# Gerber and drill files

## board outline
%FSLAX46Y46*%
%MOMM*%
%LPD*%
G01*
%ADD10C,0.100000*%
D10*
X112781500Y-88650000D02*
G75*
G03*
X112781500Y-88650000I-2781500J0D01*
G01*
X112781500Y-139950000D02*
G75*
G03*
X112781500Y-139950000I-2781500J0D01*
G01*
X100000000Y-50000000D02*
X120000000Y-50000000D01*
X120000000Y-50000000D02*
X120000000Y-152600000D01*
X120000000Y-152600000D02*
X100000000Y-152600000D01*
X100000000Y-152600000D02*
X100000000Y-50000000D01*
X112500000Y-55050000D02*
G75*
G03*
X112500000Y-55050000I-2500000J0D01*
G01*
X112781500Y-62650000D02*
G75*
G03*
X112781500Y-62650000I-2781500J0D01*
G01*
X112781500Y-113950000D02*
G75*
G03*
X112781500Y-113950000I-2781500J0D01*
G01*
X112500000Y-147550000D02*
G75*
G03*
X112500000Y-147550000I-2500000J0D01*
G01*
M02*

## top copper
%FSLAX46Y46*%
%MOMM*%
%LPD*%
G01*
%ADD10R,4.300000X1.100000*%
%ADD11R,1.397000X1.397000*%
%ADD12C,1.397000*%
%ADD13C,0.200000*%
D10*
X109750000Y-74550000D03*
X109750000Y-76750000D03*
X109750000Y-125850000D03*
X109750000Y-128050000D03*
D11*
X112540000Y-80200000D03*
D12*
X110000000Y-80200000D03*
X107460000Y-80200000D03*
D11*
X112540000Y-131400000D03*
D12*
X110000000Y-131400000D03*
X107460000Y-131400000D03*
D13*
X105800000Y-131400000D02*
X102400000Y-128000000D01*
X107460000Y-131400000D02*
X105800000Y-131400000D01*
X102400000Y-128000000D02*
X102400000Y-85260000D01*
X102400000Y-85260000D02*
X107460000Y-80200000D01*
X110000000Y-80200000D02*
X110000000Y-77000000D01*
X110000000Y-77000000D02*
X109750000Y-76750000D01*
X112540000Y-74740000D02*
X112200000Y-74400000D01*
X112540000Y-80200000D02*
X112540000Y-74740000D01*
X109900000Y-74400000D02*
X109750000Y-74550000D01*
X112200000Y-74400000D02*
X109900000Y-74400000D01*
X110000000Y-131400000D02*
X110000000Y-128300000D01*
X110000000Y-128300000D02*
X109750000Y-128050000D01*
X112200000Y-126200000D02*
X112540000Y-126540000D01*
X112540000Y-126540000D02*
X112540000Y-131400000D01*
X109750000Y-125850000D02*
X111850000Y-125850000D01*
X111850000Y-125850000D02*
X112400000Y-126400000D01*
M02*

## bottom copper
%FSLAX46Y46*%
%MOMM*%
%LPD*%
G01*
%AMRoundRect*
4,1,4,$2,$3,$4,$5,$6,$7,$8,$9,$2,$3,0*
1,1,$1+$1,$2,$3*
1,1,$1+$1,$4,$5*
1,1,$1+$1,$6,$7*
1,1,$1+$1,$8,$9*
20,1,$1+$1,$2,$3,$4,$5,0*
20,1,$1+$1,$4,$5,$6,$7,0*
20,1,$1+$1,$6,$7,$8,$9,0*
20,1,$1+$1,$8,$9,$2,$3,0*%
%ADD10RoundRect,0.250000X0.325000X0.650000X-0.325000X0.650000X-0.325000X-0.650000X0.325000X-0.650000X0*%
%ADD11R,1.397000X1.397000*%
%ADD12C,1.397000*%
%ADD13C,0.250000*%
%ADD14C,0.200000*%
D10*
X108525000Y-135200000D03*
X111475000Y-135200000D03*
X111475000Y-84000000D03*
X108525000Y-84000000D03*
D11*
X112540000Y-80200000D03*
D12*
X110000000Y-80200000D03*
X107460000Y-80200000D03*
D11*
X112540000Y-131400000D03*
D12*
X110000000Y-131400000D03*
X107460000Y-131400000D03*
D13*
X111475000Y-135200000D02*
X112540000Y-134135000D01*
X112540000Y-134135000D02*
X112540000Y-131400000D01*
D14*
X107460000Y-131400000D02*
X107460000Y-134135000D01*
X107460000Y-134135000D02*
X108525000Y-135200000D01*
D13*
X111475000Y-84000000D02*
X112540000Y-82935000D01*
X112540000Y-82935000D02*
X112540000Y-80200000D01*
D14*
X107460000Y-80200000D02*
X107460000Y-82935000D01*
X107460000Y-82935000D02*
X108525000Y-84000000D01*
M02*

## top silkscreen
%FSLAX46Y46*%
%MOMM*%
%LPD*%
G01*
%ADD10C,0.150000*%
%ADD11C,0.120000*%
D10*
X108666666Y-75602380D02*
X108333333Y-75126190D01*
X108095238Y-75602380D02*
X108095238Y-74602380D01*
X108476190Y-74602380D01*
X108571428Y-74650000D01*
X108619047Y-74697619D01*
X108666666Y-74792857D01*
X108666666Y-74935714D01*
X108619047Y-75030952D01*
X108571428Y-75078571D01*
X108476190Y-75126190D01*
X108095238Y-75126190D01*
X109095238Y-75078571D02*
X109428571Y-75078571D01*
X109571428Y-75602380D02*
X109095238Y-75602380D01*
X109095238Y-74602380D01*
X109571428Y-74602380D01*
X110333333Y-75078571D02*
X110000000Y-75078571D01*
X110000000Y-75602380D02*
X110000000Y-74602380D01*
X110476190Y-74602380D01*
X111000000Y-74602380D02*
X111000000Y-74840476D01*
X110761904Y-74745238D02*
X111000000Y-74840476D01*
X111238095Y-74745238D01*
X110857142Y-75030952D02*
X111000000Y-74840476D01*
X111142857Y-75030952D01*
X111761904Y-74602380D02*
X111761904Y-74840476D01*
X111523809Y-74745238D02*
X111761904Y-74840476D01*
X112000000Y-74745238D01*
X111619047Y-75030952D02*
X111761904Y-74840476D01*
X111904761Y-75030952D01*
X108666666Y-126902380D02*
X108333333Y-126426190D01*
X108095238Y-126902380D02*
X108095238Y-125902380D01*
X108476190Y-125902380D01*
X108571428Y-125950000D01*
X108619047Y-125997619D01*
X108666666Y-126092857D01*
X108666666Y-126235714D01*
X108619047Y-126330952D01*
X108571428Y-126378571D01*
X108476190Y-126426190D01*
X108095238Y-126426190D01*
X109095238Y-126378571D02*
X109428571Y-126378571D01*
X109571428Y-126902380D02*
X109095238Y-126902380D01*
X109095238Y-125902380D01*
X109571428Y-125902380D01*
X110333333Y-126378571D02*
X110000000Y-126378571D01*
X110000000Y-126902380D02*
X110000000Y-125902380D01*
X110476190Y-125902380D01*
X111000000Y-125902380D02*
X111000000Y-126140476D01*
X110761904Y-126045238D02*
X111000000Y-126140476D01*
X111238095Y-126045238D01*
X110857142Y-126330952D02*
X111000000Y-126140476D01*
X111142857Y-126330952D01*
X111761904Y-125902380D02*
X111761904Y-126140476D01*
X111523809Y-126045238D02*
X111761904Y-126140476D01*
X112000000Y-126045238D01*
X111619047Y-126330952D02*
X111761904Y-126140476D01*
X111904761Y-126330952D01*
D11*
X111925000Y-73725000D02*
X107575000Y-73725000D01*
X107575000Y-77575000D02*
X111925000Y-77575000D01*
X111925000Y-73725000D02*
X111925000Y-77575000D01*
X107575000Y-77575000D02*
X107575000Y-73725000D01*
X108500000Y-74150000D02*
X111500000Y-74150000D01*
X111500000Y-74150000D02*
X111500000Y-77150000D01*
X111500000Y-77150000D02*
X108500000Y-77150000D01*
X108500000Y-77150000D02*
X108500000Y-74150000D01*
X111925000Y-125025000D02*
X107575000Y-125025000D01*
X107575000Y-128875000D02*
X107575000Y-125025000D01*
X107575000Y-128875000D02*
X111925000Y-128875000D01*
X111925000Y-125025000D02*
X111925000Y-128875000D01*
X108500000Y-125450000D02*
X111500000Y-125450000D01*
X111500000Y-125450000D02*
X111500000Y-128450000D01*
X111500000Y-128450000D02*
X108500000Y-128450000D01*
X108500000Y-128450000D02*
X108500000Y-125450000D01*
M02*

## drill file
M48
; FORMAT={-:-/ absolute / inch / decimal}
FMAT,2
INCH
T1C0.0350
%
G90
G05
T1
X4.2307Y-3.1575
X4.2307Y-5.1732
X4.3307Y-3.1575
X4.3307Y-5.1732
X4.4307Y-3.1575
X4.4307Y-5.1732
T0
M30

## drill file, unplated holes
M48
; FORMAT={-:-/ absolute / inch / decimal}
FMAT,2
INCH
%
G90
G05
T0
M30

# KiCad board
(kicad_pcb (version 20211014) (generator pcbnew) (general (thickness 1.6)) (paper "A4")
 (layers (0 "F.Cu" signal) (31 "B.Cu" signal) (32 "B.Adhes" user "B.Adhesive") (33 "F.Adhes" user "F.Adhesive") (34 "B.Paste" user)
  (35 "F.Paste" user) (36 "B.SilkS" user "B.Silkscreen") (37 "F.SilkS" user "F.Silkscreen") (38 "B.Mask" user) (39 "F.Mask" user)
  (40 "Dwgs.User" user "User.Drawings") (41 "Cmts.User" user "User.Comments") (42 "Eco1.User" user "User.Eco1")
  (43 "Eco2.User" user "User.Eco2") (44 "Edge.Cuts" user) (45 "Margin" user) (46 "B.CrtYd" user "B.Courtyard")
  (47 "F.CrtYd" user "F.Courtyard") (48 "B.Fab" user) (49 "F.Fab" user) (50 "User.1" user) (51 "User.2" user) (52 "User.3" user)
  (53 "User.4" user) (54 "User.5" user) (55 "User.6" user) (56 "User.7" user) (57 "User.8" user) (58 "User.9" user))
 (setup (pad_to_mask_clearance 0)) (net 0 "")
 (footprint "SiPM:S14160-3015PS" (layer "F.Cu") (at 110 75.65)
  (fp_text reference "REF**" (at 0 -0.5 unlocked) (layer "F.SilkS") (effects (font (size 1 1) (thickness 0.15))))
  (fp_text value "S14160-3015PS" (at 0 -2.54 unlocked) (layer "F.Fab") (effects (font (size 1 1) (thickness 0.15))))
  (fp_line (start 1.925 -1.925) (end -2.425 -1.925) (layer "F.SilkS") (width 0.12))
  (fp_line (start -2.425 1.925) (end 1.925 1.925) (layer "F.SilkS") (width 0.12))
  (fp_line (start 1.925 -1.925) (end 1.925 1.925) (layer "F.SilkS") (width 0.12))
  (fp_line (start -2.425 1.925) (end -2.425 -1.925) (layer "F.SilkS") (width 0.12))
  (fp_rect (start -1.5 -1.5) (end 1.5 1.5) (layer "F.SilkS") (width 0.12) (fill none))
  (pad "1" smd rect (at -0.25 -1.1) (size 4.3 1.1) (layers "F.Cu" "F.Paste" "F.Mask"))
  (pad "2" smd rect (at -0.25 1.1) (size 4.3 1.1) (layers "F.Cu" "F.Paste" "F.Mask")))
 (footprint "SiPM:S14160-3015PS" (layer "F.Cu") (at 110 126.95)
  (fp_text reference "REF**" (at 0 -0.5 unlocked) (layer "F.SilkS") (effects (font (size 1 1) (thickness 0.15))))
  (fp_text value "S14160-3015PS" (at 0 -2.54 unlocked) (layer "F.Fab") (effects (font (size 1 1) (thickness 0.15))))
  (fp_line (start 1.925 -1.925) (end -2.425 -1.925) (layer "F.SilkS") (width 0.12))
  (fp_line (start -2.425 1.925) (end -2.425 -1.925) (layer "F.SilkS") (width 0.12))
  (fp_line (start -2.425 1.925) (end 1.925 1.925) (layer "F.SilkS") (width 0.12))
  (fp_line (start 1.925 -1.925) (end 1.925 1.925) (layer "F.SilkS") (width 0.12))
  (fp_rect (start -1.5 -1.5) (end 1.5 1.5) (layer "F.SilkS") (width 0.12) (fill none))
  (pad "1" smd rect (at -0.25 -1.1) (size 4.3 1.1) (layers "F.Cu" "F.Paste" "F.Mask"))
  (pad "2" smd rect (at -0.25 1.1) (size 4.3 1.1) (layers "F.Cu" "F.Paste" "F.Mask")))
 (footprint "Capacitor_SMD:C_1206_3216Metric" (layer "B.Cu") (at 110 84 180)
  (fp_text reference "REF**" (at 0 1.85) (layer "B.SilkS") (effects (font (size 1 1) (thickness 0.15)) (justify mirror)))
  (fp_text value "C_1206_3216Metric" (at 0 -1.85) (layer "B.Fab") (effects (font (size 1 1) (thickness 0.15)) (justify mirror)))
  (pad "1" smd roundrect (at -1.475 0 180) (size 1.15 1.8) (layers "B.Cu" "B.Paste" "B.Mask") (roundrect_rratio 0.2173913043))
  (pad "2" smd roundrect (at 1.475 0 180) (size 1.15 1.8) (layers "B.Cu" "B.Paste" "B.Mask") (roundrect_rratio 0.2173913043)))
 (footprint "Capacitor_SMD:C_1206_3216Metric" (layer "B.Cu") (at 110 135.2 180)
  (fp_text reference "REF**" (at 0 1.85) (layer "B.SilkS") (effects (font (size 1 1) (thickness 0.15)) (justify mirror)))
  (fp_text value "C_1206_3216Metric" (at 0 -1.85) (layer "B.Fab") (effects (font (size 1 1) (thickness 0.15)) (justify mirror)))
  (pad "1" smd roundrect (at -1.475 0 180) (size 1.15 1.8) (layers "B.Cu" "B.Paste" "B.Mask") (roundrect_rratio 0.2173913043))
  (pad "2" smd roundrect (at 1.475 0 180) (size 1.15 1.8) (layers "B.Cu" "B.Paste" "B.Mask") (roundrect_rratio 0.2173913043)))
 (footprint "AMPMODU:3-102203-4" (layer "B.Cu") (at 112.54 80.2 180)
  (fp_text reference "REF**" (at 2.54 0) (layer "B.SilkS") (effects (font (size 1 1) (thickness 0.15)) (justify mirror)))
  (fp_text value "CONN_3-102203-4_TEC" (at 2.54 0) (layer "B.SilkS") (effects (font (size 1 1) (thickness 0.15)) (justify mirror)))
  (pad "1" thru_hole rect locked (at 0 0 180) (size 1.397 1.397) (drill 0.889) (layers *.Cu *.Mask))
  (pad "2" thru_hole circle locked (at 2.54 0 180) (size 1.397 1.397) (drill 0.889) (layers *.Cu *.Mask))
  (pad "3" thru_hole circle locked (at 5.08 0 180) (size 1.397 1.397) (drill 0.889) (layers *.Cu *.Mask)))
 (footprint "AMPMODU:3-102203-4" (layer "B.Cu") (at 112.54 131.4 180)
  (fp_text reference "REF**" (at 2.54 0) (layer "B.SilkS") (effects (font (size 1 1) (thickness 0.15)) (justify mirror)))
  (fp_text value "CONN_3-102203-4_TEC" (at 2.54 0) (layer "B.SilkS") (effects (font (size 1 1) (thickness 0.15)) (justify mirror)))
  (pad "1" thru_hole rect locked (at 0 0 180) (size 1.397 1.397) (drill 0.889) (layers *.Cu *.Mask))
  (pad "2" thru_hole circle locked (at 2.54 0 180) (size 1.397 1.397) (drill 0.889) (layers *.Cu *.Mask))
  (pad "3" thru_hole circle locked (at 5.08 0 180) (size 1.397 1.397) (drill 0.889) (layers *.Cu *.Mask)))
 (gr_circle (center 110 88.65) (end 112.7815 88.65) (layer "Edge.Cuts") (width 0.1) (fill none))
 (gr_circle (center 110 139.95) (end 112.7815 139.95) (layer "Edge.Cuts") (width 0.1) (fill none))
 (gr_rect (start 100 50) (end 120 152.6) (layer "Edge.Cuts") (width 0.1) (fill none))
 (gr_circle (center 110 55.05) (end 112.5 55.05) (layer "Edge.Cuts") (width 0.1) (fill none))
 (gr_circle (center 110 62.65) (end 112.7815 62.65) (layer "Edge.Cuts") (width 0.1) (fill none))
 (gr_circle (center 110 113.95) (end 112.7815 113.95) (layer "Edge.Cuts") (width 0.1) (fill none))
 (gr_circle (center 110 147.55) (end 112.5 147.55) (layer "Edge.Cuts") (width 0.1) (fill none))
 (segment (start 107.46 131.4) (end 105.8 131.4) (width 0.2) (layer "F.Cu") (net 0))
 (segment (start 112.54 126.54) (end 112.54 131.4) (width 0.2) (layer "F.Cu") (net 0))
 (segment (start 102.4 128) (end 102.4 85.26) (width 0.2) (layer "F.Cu") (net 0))
 (segment (start 112.54 80.2) (end 112.54 74.74) (width 0.2) (layer "F.Cu") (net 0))
 (segment (start 112.2 74.4) (end 109.9 74.4) (width 0.2) (layer "F.Cu") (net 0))
 (segment (start 112.2 126.2) (end 112.54 126.54) (width 0.2) (layer "F.Cu") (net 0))
 (segment (start 110 128.3) (end 109.75 128.05) (width 0.2) (layer "F.Cu") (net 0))
 (segment (start 112.54 74.74) (end 112.2 74.4) (width 0.2) (layer "F.Cu") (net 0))
 (segment (start 110 80.2) (end 110 77) (width 0.2) (layer "F.Cu") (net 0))
 (segment (start 109.75 125.85) (end 111.85 125.85) (width 0.2) (layer "F.Cu") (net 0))
 (segment (start 111.85 125.85) (end 112.4 126.4) (width 0.2) (layer "F.Cu") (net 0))
 (segment (start 110 131.4) (end 110 128.3) (width 0.2) (layer "F.Cu") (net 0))
 (segment (start 110 77) (end 109.75 76.75) (width 0.2) (layer "F.Cu") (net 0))
 (segment (start 102.4 85.26) (end 107.46 80.2) (width 0.2) (layer "F.Cu") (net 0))
 (segment (start 109.9 74.4) (end 109.75 74.55) (width 0.2) (layer "F.Cu") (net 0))
 (segment (start 105.8 131.4) (end 102.4 128) (width 0.2) (layer "F.Cu") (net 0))
 (segment (start 111.475 84) (end 112.54 82.935) (width 0.25) (layer "B.Cu") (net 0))
 (segment (start 111.475 135.2) (end 112.54 134.135) (width 0.25) (layer "B.Cu") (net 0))
 (segment (start 107.46 131.4) (end 107.46 134.135) (width 0.2) (layer "B.Cu") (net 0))
 (segment (start 107.46 134.135) (end 108.525 135.2) (width 0.2) (layer "B.Cu") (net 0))
 (segment (start 112.54 134.135) (end 112.54 131.4) (width 0.25) (layer "B.Cu") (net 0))
 (segment (start 112.54 82.935) (end 112.54 80.2) (width 0.25) (layer "B.Cu") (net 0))
 (segment (start 107.46 80.2) (end 107.46 82.935) (width 0.2) (layer "B.Cu") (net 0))
 (segment (start 107.46 82.935) (end 108.525 84) (width 0.2) (layer "B.Cu") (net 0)))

